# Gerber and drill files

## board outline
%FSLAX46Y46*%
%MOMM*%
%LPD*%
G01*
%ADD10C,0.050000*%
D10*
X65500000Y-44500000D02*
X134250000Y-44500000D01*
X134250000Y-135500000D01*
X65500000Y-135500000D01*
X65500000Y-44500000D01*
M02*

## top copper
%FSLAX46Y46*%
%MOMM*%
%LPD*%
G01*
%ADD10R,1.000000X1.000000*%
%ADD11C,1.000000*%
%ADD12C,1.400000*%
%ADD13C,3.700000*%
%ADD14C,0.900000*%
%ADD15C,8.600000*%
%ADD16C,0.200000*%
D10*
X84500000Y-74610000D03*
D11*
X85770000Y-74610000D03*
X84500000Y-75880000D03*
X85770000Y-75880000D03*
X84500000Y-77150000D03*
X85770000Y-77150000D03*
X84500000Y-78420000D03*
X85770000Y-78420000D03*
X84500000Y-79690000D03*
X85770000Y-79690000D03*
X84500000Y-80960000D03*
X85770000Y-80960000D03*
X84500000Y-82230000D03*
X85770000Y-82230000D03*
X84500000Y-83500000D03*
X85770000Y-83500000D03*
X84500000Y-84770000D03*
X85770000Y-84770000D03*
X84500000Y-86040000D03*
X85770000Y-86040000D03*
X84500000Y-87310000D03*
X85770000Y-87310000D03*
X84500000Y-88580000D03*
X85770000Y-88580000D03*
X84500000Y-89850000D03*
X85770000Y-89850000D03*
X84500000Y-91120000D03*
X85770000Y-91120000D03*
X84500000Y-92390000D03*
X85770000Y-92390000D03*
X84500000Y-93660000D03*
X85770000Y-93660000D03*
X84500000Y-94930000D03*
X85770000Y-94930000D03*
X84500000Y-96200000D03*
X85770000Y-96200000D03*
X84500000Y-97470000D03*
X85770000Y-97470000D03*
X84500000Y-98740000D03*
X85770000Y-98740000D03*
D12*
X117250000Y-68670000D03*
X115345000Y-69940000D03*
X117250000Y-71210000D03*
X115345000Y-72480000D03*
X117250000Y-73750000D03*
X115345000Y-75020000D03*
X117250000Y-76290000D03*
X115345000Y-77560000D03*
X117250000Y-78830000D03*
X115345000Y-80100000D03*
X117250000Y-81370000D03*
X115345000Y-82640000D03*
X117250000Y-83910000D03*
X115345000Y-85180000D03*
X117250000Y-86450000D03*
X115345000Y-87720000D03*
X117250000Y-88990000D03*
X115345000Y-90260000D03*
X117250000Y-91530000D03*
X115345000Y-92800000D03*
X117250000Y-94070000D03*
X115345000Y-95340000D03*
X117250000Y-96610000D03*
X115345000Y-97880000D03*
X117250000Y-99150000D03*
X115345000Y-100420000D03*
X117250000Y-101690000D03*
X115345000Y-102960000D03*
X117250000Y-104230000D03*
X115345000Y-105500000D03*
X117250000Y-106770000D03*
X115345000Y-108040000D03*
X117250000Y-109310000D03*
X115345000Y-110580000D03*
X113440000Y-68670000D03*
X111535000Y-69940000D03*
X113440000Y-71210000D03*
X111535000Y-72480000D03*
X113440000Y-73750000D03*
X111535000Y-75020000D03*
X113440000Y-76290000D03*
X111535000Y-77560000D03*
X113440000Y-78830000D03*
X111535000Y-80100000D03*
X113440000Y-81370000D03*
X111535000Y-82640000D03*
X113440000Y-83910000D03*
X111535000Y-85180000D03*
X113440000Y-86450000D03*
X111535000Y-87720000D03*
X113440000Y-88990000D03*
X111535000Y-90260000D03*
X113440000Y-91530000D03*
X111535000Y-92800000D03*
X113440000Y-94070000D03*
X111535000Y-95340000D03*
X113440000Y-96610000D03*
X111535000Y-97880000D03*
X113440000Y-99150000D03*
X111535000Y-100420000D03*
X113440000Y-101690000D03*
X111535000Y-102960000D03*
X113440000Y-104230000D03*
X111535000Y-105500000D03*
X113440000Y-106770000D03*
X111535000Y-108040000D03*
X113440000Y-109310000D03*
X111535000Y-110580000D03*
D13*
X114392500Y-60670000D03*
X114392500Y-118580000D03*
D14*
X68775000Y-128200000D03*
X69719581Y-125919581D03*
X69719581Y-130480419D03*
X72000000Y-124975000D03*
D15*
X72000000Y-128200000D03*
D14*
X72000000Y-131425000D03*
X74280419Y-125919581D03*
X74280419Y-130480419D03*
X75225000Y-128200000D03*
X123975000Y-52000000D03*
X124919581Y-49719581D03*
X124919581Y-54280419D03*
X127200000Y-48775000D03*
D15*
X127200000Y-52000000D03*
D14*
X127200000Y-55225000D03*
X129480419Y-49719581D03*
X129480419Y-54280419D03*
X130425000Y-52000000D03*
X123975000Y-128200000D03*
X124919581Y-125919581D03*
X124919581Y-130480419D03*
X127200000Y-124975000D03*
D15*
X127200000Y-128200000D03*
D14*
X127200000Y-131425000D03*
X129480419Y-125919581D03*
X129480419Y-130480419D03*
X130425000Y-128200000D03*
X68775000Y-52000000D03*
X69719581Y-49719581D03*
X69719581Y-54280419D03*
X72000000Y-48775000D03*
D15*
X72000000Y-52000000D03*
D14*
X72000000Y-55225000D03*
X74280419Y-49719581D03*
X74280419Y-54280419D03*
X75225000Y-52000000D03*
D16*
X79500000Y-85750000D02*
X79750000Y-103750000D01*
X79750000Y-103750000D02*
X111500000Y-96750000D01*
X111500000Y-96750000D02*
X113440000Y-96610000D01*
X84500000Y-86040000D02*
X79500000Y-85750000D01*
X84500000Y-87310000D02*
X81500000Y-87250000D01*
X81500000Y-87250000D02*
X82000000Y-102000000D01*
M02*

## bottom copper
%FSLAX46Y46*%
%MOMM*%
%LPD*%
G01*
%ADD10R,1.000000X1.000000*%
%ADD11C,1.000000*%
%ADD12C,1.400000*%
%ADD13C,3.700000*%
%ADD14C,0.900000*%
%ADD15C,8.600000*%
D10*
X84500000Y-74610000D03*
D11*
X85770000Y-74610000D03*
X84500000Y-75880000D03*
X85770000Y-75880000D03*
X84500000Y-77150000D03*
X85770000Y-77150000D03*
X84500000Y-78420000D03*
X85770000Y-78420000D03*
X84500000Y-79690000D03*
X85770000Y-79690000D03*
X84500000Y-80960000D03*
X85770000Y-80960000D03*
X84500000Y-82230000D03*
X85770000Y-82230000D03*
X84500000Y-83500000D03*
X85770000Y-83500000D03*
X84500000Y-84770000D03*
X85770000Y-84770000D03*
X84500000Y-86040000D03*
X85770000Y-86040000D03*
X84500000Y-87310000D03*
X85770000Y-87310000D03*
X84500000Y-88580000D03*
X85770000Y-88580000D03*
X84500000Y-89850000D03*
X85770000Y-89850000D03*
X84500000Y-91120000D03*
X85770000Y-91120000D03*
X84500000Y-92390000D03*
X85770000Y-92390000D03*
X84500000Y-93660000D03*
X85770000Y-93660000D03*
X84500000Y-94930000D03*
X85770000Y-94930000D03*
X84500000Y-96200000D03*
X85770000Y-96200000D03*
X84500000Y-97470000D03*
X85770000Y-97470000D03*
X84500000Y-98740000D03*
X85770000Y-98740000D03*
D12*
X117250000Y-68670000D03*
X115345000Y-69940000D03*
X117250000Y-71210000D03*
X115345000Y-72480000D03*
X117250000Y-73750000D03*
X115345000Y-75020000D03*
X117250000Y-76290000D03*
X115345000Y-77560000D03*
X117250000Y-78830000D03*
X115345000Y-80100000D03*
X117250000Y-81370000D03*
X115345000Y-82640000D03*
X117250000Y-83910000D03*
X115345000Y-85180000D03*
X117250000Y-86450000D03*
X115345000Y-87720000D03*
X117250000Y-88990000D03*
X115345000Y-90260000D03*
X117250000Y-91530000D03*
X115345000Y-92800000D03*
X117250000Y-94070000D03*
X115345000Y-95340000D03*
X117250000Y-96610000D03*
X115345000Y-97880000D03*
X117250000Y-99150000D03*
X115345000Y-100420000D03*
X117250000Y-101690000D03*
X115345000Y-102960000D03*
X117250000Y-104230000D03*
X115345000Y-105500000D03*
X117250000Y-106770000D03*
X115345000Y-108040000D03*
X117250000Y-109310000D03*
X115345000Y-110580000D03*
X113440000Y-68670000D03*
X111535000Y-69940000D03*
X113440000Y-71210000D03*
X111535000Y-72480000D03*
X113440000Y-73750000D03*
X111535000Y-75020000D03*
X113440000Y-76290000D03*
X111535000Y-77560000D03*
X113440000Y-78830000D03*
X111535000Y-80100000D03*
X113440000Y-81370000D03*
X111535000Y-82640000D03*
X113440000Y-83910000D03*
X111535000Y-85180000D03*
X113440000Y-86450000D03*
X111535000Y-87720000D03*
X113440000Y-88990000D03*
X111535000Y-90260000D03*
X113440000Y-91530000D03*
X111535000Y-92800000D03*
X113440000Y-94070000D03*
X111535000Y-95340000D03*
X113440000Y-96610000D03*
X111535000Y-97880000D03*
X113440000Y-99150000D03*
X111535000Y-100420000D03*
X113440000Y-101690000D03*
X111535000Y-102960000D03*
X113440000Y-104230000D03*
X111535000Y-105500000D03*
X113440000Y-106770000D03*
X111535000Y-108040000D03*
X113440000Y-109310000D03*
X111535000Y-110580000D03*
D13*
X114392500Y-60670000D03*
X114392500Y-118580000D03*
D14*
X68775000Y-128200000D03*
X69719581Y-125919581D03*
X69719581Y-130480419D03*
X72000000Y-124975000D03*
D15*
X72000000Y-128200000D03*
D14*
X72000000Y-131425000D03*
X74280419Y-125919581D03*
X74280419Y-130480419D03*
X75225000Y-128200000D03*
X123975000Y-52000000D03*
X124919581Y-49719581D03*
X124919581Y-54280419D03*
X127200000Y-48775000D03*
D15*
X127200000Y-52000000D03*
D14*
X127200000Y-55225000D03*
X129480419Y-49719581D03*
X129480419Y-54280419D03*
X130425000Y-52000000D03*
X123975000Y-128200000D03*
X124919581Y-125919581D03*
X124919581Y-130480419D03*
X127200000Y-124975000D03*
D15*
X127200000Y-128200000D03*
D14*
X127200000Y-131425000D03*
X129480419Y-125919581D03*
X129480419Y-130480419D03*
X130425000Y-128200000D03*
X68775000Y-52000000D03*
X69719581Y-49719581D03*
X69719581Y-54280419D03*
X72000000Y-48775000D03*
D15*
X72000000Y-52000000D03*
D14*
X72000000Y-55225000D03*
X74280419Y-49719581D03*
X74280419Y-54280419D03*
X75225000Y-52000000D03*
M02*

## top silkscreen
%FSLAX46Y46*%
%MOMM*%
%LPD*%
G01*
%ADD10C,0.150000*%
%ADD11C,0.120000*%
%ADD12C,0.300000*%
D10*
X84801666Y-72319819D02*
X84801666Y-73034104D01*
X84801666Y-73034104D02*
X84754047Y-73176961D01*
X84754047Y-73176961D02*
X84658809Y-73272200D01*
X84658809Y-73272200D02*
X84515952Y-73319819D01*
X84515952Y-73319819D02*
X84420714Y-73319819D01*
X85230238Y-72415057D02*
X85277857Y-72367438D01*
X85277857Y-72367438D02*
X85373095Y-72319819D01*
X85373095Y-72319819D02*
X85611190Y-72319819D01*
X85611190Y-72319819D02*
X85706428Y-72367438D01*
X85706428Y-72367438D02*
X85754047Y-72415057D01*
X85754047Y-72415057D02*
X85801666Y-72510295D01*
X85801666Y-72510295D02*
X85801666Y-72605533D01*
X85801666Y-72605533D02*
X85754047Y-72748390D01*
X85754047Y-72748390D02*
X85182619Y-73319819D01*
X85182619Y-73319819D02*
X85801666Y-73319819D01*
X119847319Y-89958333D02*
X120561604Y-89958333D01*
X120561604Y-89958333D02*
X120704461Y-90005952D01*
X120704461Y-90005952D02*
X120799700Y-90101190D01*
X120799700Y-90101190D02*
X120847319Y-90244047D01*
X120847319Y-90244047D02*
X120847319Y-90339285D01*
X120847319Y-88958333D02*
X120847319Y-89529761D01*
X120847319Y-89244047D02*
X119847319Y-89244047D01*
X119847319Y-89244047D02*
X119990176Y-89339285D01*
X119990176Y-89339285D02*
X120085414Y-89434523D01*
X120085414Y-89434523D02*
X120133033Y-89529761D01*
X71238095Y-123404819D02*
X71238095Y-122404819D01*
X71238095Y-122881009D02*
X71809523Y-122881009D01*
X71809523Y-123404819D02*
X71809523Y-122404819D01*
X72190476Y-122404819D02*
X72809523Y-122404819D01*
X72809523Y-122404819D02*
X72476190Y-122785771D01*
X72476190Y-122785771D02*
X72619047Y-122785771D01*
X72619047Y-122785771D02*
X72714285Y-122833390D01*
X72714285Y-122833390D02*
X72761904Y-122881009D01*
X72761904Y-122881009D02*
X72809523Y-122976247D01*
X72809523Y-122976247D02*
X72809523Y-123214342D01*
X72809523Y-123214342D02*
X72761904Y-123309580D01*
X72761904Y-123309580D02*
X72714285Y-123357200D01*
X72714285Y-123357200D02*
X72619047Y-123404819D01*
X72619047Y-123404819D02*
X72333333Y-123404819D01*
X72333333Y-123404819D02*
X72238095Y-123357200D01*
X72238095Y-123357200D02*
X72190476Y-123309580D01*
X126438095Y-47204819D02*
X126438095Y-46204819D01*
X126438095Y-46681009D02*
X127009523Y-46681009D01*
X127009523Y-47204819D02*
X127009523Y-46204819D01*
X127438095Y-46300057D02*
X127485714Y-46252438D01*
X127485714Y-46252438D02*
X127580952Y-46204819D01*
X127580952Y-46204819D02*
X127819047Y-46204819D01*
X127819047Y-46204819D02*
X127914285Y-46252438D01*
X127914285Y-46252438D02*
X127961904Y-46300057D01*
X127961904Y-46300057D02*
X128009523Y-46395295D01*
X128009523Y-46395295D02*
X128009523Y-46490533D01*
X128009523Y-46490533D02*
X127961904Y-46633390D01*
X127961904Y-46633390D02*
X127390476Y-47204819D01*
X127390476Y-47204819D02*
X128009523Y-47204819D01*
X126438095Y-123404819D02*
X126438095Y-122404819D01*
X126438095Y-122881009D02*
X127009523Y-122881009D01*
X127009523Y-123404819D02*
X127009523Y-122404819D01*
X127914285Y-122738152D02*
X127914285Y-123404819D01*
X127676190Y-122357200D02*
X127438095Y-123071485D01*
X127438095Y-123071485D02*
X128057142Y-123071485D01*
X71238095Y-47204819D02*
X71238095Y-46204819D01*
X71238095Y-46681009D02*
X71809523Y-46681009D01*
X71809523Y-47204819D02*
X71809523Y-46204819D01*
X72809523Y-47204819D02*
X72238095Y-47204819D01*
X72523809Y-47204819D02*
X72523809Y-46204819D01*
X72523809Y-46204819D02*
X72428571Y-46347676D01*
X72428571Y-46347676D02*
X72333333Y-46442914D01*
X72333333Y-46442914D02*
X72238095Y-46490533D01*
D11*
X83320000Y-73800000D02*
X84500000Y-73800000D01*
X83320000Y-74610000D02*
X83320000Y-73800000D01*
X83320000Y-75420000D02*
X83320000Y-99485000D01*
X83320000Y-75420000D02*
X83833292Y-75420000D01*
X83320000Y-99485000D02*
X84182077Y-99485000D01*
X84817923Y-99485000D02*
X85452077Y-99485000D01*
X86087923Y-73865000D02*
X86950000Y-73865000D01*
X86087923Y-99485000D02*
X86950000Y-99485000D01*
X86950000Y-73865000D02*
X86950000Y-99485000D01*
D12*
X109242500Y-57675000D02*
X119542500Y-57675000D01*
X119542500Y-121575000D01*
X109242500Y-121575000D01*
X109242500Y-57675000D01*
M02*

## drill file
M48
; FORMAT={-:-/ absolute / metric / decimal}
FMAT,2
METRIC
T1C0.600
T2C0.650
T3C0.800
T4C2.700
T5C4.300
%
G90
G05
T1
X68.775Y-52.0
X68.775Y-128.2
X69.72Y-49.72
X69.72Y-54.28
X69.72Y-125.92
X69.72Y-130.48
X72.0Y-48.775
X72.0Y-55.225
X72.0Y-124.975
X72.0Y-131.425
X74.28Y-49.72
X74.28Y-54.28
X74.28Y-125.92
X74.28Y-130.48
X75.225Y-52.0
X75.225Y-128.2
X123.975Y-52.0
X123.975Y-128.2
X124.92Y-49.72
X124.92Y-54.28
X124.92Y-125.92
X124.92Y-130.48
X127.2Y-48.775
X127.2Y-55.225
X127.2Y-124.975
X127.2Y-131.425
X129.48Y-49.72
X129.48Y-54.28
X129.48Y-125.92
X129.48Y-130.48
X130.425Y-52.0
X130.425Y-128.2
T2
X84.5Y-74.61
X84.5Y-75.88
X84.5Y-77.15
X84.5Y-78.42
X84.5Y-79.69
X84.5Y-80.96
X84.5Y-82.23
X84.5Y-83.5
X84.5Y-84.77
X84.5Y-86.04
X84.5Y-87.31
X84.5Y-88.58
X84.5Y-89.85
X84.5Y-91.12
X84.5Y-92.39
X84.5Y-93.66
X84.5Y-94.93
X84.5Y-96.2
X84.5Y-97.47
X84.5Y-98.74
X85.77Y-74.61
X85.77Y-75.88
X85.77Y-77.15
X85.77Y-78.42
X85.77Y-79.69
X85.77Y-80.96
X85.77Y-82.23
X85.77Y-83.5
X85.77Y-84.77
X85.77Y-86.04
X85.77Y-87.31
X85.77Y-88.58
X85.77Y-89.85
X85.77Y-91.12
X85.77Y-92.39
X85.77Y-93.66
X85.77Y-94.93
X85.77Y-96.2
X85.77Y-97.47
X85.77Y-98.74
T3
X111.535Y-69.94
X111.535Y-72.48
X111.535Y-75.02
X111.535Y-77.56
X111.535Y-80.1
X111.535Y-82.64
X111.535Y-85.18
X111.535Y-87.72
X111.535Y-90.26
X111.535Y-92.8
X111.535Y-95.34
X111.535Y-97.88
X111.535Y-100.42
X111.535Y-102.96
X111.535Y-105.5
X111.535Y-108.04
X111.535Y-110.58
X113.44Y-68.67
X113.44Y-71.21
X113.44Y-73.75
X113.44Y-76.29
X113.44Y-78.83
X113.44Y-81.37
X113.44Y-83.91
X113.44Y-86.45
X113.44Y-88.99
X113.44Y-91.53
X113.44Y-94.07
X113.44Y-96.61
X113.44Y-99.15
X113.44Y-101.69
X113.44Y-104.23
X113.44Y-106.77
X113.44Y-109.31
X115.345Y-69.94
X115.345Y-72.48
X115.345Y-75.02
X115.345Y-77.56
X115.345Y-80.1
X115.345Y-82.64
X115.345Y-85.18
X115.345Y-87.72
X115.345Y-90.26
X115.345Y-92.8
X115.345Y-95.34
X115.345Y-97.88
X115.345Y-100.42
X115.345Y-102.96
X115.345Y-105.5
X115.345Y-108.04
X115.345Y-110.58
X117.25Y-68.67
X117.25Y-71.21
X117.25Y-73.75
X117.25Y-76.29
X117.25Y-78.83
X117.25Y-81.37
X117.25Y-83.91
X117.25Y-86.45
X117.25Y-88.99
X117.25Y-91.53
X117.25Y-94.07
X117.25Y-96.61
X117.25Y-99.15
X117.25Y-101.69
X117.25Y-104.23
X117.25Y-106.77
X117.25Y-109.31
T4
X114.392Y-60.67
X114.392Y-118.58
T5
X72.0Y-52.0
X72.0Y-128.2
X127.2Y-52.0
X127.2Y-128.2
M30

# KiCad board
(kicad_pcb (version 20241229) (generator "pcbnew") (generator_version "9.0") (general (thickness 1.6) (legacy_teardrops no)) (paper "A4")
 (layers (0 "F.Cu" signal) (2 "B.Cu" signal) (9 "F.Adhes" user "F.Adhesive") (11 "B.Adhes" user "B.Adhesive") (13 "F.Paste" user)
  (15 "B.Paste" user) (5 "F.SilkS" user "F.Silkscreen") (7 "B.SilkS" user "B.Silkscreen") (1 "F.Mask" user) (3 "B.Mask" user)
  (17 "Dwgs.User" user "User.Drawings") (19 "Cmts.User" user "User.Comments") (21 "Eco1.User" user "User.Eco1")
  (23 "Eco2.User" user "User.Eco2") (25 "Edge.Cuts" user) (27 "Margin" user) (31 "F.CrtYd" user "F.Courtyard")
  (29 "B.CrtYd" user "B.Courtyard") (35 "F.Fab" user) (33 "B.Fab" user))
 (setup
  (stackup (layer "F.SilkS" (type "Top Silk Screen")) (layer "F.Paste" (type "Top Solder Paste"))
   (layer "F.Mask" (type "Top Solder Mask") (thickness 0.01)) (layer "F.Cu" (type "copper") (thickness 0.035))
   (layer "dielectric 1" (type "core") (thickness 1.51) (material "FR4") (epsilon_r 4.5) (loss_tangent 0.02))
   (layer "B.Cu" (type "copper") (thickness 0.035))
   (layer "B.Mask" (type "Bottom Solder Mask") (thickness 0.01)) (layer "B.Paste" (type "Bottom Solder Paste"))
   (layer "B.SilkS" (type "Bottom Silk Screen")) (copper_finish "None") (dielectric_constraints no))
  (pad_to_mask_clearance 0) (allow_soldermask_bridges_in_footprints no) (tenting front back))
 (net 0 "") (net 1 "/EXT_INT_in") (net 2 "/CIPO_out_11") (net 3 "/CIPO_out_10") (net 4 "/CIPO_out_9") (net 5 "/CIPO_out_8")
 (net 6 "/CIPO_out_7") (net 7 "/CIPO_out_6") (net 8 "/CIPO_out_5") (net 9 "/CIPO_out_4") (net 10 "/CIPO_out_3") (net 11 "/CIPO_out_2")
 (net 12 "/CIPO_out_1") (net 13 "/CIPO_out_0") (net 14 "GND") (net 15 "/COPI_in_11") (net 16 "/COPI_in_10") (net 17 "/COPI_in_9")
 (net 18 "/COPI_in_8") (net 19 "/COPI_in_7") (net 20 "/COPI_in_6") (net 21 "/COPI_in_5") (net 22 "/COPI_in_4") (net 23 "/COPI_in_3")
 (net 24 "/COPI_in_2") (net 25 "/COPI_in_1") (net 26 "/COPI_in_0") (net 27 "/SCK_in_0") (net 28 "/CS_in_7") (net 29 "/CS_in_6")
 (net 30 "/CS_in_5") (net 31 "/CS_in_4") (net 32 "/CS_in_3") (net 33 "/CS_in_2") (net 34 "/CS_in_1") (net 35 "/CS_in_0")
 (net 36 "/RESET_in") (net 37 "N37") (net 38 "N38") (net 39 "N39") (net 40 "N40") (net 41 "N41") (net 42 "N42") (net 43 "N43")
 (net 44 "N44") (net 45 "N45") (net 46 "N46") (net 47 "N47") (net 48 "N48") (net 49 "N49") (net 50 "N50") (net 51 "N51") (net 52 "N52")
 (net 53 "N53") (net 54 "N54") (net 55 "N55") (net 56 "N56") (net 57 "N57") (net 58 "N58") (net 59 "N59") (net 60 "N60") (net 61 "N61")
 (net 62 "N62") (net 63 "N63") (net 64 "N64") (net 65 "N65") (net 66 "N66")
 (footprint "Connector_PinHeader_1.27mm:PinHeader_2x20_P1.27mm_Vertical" (layer "F.Cu") (at 84.5 74.61)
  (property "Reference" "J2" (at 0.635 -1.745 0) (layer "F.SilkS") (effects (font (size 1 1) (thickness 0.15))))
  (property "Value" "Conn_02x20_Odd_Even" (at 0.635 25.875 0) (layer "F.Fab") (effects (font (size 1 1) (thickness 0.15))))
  (fp_line (start -1.18 -0.81) (end 0 -0.81) (stroke (width 0.12) (type solid)) (layer "F.SilkS"))
  (fp_line (start -1.18 0) (end -1.18 -0.81) (stroke (width 0.12) (type solid)) (layer "F.SilkS"))
  (fp_line (start -1.18 0.81) (end -1.18 24.875) (stroke (width 0.12) (type solid)) (layer "F.SilkS"))
  (fp_line (start -1.18 0.81) (end -0.666708 0.81) (stroke (width 0.12) (type solid)) (layer "F.SilkS"))
  (fp_line (start -1.18 24.875) (end -0.317923 24.875) (stroke (width 0.12) (type solid)) (layer "F.SilkS"))
  (fp_line (start 0.317923 24.875) (end 0.952077 24.875) (stroke (width 0.12) (type solid)) (layer "F.SilkS"))
  (fp_line (start 1.587923 -0.745) (end 2.45 -0.745) (stroke (width 0.12) (type solid)) (layer "F.SilkS"))
  (fp_line (start 1.587923 24.875) (end 2.45 24.875) (stroke (width 0.12) (type solid)) (layer "F.SilkS"))
  (fp_line (start 2.45 -0.745) (end 2.45 24.875) (stroke (width 0.12) (type solid)) (layer "F.SilkS"))
  (pad "1" thru_hole rect (at 0 0) (size 1 1) (drill 0.65) (layers "*.Cu" "*.Mask") (remove_unused_layers no) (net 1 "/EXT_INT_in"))
  (pad "2" thru_hole circle (at 1.27 0) (size 1 1) (drill 0.65) (layers "*.Cu" "*.Mask") (remove_unused_layers no) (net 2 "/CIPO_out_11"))
  (pad "3" thru_hole circle (at 0 1.27) (size 1 1) (drill 0.65) (layers "*.Cu" "*.Mask") (remove_unused_layers no) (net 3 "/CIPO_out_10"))
  (pad "4" thru_hole circle (at 1.27 1.27) (size 1 1) (drill 0.65) (layers "*.Cu" "*.Mask") (remove_unused_layers no) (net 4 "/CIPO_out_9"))
  (pad "5" thru_hole circle (at 0 2.54) (size 1 1) (drill 0.65) (layers "*.Cu" "*.Mask") (remove_unused_layers no) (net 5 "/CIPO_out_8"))
  (pad "6" thru_hole circle (at 1.27 2.54) (size 1 1) (drill 0.65) (layers "*.Cu" "*.Mask") (remove_unused_layers no) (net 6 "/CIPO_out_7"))
  (pad "7" thru_hole circle (at 0 3.81) (size 1 1) (drill 0.65) (layers "*.Cu" "*.Mask") (remove_unused_layers no) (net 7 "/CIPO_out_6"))
  (pad "8" thru_hole circle (at 1.27 3.81) (size 1 1) (drill 0.65) (layers "*.Cu" "*.Mask") (remove_unused_layers no) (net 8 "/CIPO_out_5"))
  (pad "9" thru_hole circle (at 0 5.08) (size 1 1) (drill 0.65) (layers "*.Cu" "*.Mask") (remove_unused_layers no) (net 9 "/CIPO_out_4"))
  (pad "10" thru_hole circle (at 1.27 5.08) (size 1 1) (drill 0.65) (layers "*.Cu" "*.Mask") (remove_unused_layers no)
   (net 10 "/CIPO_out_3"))
  (pad "11" thru_hole circle (at 0 6.35) (size 1 1) (drill 0.65) (layers "*.Cu" "*.Mask") (remove_unused_layers no) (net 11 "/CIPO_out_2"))
  (pad "12" thru_hole circle (at 1.27 6.35) (size 1 1) (drill 0.65) (layers "*.Cu" "*.Mask") (remove_unused_layers no)
   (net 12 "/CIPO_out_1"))
  (pad "13" thru_hole circle (at 0 7.62) (size 1 1) (drill 0.65) (layers "*.Cu" "*.Mask") (remove_unused_layers no) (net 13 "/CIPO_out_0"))
  (pad "14" thru_hole circle (at 1.27 7.62) (size 1 1) (drill 0.65) (layers "*.Cu" "*.Mask") (remove_unused_layers no) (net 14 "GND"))
  (pad "15" thru_hole circle (at 0 8.89) (size 1 1) (drill 0.65) (layers "*.Cu" "*.Mask") (remove_unused_layers no) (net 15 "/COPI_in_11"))
  (pad "16" thru_hole circle (at 1.27 8.89) (size 1 1) (drill 0.65) (layers "*.Cu" "*.Mask") (remove_unused_layers no)
   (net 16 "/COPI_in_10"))
  (pad "17" thru_hole circle (at 0 10.16) (size 1 1) (drill 0.65) (layers "*.Cu" "*.Mask") (remove_unused_layers no) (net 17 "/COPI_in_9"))
  (pad "18" thru_hole circle (at 1.27 10.16) (size 1 1) (drill 0.65) (layers "*.Cu" "*.Mask") (remove_unused_layers no)
   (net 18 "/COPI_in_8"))
  (pad "19" thru_hole circle (at 0 11.43) (size 1 1) (drill 0.65) (layers "*.Cu" "*.Mask") (remove_unused_layers no) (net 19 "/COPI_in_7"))
  (pad "20" thru_hole circle (at 1.27 11.43) (size 1 1) (drill 0.65) (layers "*.Cu" "*.Mask") (remove_unused_layers no)
   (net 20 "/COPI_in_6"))
  (pad "21" thru_hole circle (at 0 12.7) (size 1 1) (drill 0.65) (layers "*.Cu" "*.Mask") (remove_unused_layers no) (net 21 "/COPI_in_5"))
  (pad "22" thru_hole circle (at 1.27 12.7) (size 1 1) (drill 0.65) (layers "*.Cu" "*.Mask") (remove_unused_layers no) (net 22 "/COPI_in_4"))
  (pad "23" thru_hole circle (at 0 13.97) (size 1 1) (drill 0.65) (layers "*.Cu" "*.Mask") (remove_unused_layers no) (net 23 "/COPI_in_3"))
  (pad "24" thru_hole circle (at 1.27 13.97) (size 1 1) (drill 0.65) (layers "*.Cu" "*.Mask") (remove_unused_layers no)
   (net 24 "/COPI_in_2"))
  (pad "25" thru_hole circle (at 0 15.24) (size 1 1) (drill 0.65) (layers "*.Cu" "*.Mask") (remove_unused_layers no) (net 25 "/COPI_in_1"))
  (pad "26" thru_hole circle (at 1.27 15.24) (size 1 1) (drill 0.65) (layers "*.Cu" "*.Mask") (remove_unused_layers no)
   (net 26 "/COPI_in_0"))
  (pad "27" thru_hole circle (at 0 16.51) (size 1 1) (drill 0.65) (layers "*.Cu" "*.Mask") (remove_unused_layers no) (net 14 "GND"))
  (pad "28" thru_hole circle (at 1.27 16.51) (size 1 1) (drill 0.65) (layers "*.Cu" "*.Mask") (remove_unused_layers no) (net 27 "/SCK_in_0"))
  (pad "29" thru_hole circle (at 0 17.78) (size 1 1) (drill 0.65) (layers "*.Cu" "*.Mask") (remove_unused_layers no) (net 14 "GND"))
  (pad "30" thru_hole circle (at 1.27 17.78) (size 1 1) (drill 0.65) (layers "*.Cu" "*.Mask") (remove_unused_layers no) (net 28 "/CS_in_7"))
  (pad "31" thru_hole circle (at 0 19.05) (size 1 1) (drill 0.65) (layers "*.Cu" "*.Mask") (remove_unused_layers no) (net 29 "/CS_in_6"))
  (pad "32" thru_hole circle (at 1.27 19.05) (size 1 1) (drill 0.65) (layers "*.Cu" "*.Mask") (remove_unused_layers no) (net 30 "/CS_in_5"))
  (pad "33" thru_hole circle (at 0 20.32) (size 1 1) (drill 0.65) (layers "*.Cu" "*.Mask") (remove_unused_layers no) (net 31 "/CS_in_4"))
  (pad "34" thru_hole circle (at 1.27 20.32) (size 1 1) (drill 0.65) (layers "*.Cu" "*.Mask") (remove_unused_layers no) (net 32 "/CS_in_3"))
  (pad "35" thru_hole circle (at 0 21.59) (size 1 1) (drill 0.65) (layers "*.Cu" "*.Mask") (remove_unused_layers no) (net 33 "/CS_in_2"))
  (pad "36" thru_hole circle (at 1.27 21.59) (size 1 1) (drill 0.65) (layers "*.Cu" "*.Mask") (remove_unused_layers no) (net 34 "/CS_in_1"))
  (pad "37" thru_hole circle (at 0 22.86) (size 1 1) (drill 0.65) (layers "*.Cu" "*.Mask") (remove_unused_layers no) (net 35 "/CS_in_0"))
  (pad "38" thru_hole circle (at 1.27 22.86) (size 1 1) (drill 0.65) (layers "*.Cu" "*.Mask") (remove_unused_layers no) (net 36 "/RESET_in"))
  (pad "39" thru_hole circle (at 0 24.13) (size 1 1) (drill 0.65) (layers "*.Cu" "*.Mask") (remove_unused_layers no) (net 14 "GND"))
  (pad "40" thru_hole circle (at 1.27 24.13) (size 1 1) (drill 0.65) (layers "*.Cu" "*.Mask") (remove_unused_layers no) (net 14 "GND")))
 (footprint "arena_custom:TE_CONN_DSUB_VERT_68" (layer "F.Cu") (at 114.3925 89.625 -90)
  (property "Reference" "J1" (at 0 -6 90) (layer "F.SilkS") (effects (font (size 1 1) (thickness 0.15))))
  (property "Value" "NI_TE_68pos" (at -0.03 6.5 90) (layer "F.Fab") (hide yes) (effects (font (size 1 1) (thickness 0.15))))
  (fp_rect (start -31.95 -5.15) (end 31.95 5.15) (stroke (width 0.3) (type default)) (fill no) (layer "F.SilkS"))
  (pad "1" thru_hole circle (at -20.955 -2.8575 270) (size 1.4 1.4) (drill 0.8) (layers "*.Cu" "*.Mask") (remove_unused_layers no)
   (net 14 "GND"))
  (pad "2" thru_hole circle (at -19.685 -0.9525 270) (size 1.4 1.4) (drill 0.8) (layers "*.Cu" "*.Mask") (remove_unused_layers no)
   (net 14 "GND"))
  (pad "3" thru_hole circle (at -18.415 -2.8575 270) (size 1.4 1.4) (drill 0.8) (layers "*.Cu" "*.Mask") (remove_unused_layers no)
   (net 14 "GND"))
  (pad "4" thru_hole circle (at -17.145 -0.9525 270) (size 1.4 1.4) (drill 0.8) (layers "*.Cu" "*.Mask") (remove_unused_layers no)
   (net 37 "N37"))
  (pad "5" thru_hole circle (at -15.875 -2.8575 270) (size 1.4 1.4) (drill 0.8) (layers "*.Cu" "*.Mask") (remove_unused_layers no)
   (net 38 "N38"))
  (pad "6" thru_hole circle (at -14.605 -0.9525 270) (size 1.4 1.4) (drill 0.8) (layers "*.Cu" "*.Mask") (remove_unused_layers no)
   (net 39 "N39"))
  (pad "7" thru_hole circle (at -13.335 -2.8575 270) (size 1.4 1.4) (drill 0.8) (layers "*.Cu" "*.Mask") (remove_unused_layers no)
   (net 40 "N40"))
  (pad "8" thru_hole circle (at -12.065 -0.9525 270) (size 1.4 1.4) (drill 0.8) (layers "*.Cu" "*.Mask") (remove_unused_layers no)
   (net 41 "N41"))
  (pad "9" thru_hole circle (at -10.795 -2.8575 270) (size 1.4 1.4) (drill 0.8) (layers "*.Cu" "*.Mask") (remove_unused_layers no)
   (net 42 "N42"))
  (pad "10" thru_hole circle (at -9.525 -0.9525 270) (size 1.4 1.4) (drill 0.8) (layers "*.Cu" "*.Mask") (remove_unused_layers no)
   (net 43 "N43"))
  (pad "11" thru_hole circle (at -8.255 -2.8575 270) (size 1.4 1.4) (drill 0.8) (layers "*.Cu" "*.Mask") (remove_unused_layers no)
   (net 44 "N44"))
  (pad "12" thru_hole circle (at -6.985 -0.9525 270) (size 1.4 1.4) (drill 0.8) (layers "*.Cu" "*.Mask") (remove_unused_layers no)
   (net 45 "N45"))
  (pad "13" thru_hole circle (at -5.715 -2.8575 270) (size 1.4 1.4) (drill 0.8) (layers "*.Cu" "*.Mask") (remove_unused_layers no)
   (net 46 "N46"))
  (pad "14" thru_hole circle (at -4.445 -0.9525 270) (size 1.4 1.4) (drill 0.8) (layers "*.Cu" "*.Mask") (remove_unused_layers no)
   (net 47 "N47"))
  (pad "15" thru_hole circle (at -3.175 -2.8575 270) (size 1.4 1.4) (drill 0.8) (layers "*.Cu" "*.Mask") (remove_unused_layers no)
   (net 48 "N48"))
  (pad "16" thru_hole circle (at -1.905 -0.9525 270) (size 1.4 1.4) (drill 0.8) (layers "*.Cu" "*.Mask") (remove_unused_layers no)
   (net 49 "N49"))
  (pad "17" thru_hole circle (at -0.635 -2.8575 270) (size 1.4 1.4) (drill 0.8) (layers "*.Cu" "*.Mask") (remove_unused_layers no)
   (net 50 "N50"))
  (pad "18" thru_hole circle (at 0.635 -0.9525 270) (size 1.4 1.4) (drill 0.8) (layers "*.Cu" "*.Mask") (remove_unused_layers no)
   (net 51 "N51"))
  (pad "19" thru_hole circle (at 1.905 -2.8575 270) (size 1.4 1.4) (drill 0.8) (layers "*.Cu" "*.Mask") (remove_unused_layers no)
   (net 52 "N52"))
  (pad "20" thru_hole circle (at 3.175 -0.9525 270) (size 1.4 1.4) (drill 0.8) (layers "*.Cu" "*.Mask") (remove_unused_layers no)
   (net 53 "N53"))
  (pad "21" thru_hole circle (at 4.445 -2.8575 270) (size 1.4 1.4) (drill 0.8) (layers "*.Cu" "*.Mask") (remove_unused_layers no)
   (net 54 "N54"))
  (pad "22" thru_hole circle (at 5.715 -0.9525 270) (size 1.4 1.4) (drill 0.8) (layers "*.Cu" "*.Mask") (remove_unused_layers no)
   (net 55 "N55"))
  (pad "23" thru_hole circle (at 6.985 -2.8575 270) (size 1.4 1.4) (drill 0.8) (layers "*.Cu" "*.Mask") (remove_unused_layers no)
   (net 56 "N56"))
  (pad "24" thru_hole circle (at 8.255 -0.9525 270) (size 1.4 1.4) (drill 0.8) (layers "*.Cu" "*.Mask") (remove_unused_layers no)
   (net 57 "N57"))
  (pad "25" thru_hole circle (at 9.525 -2.8575 270) (size 1.4 1.4) (drill 0.8) (layers "*.Cu" "*.Mask") (remove_unused_layers no)
   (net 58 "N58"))
  (pad "26" thru_hole circle (at 10.795 -0.9525 270) (size 1.4 1.4) (drill 0.8) (layers "*.Cu" "*.Mask") (remove_unused_layers no)
   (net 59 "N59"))
  (pad "27" thru_hole circle (at 12.065 -2.8575 270) (size 1.4 1.4) (drill 0.8) (layers "*.Cu" "*.Mask") (remove_unused_layers no)
   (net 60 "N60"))
  (pad "28" thru_hole circle (at 13.335 -0.9525 270) (size 1.4 1.4) (drill 0.8) (layers "*.Cu" "*.Mask") (remove_unused_layers no)
   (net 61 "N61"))
  (pad "29" thru_hole circle (at 14.605 -2.8575 270) (size 1.4 1.4) (drill 0.8) (layers "*.Cu" "*.Mask") (remove_unused_layers no)
   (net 22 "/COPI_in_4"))
  (pad "30" thru_hole circle (at 15.875 -0.9525 270) (size 1.4 1.4) (drill 0.8) (layers "*.Cu" "*.Mask") (remove_unused_layers no)
   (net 23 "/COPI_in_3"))
  (pad "31" thru_hole circle (at 17.145 -2.8575 270) (size 1.4 1.4) (drill 0.8) (layers "*.Cu" "*.Mask") (remove_unused_layers no)
   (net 24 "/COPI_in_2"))
  (pad "32" thru_hole circle (at 18.415 -0.9525 270) (size 1.4 1.4) (drill 0.8) (layers "*.Cu" "*.Mask") (remove_unused_layers no)
   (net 25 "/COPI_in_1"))
  (pad "33" thru_hole circle (at 19.685 -2.8575 270) (size 1.4 1.4) (drill 0.8) (layers "*.Cu" "*.Mask") (remove_unused_layers no)
   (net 26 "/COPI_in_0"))
  (pad "34" thru_hole circle (at 20.955 -0.9525 270) (size 1.4 1.4) (drill 0.8) (layers "*.Cu" "*.Mask") (remove_unused_layers no)
   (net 36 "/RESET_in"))
  (pad "35" thru_hole circle (at -20.955 0.9525 270) (size 1.4 1.4) (drill 0.8) (layers "*.Cu" "*.Mask") (remove_unused_layers no)
   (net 35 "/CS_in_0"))
  (pad "36" thru_hole circle (at -19.685 2.8575 270) (size 1.4 1.4) (drill 0.8) (layers "*.Cu" "*.Mask") (remove_unused_layers no)
   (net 34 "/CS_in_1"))
  (pad "37" thru_hole circle (at -18.415 0.9525 270) (size 1.4 1.4) (drill 0.8) (layers "*.Cu" "*.Mask") (remove_unused_layers no)
   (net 33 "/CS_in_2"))
  (pad "38" thru_hole circle (at -17.145 2.8575 270) (size 1.4 1.4) (drill 0.8) (layers "*.Cu" "*.Mask") (remove_unused_layers no)
   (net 32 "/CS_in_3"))
  (pad "39" thru_hole circle (at -15.875 0.9525 270) (size 1.4 1.4) (drill 0.8) (layers "*.Cu" "*.Mask") (remove_unused_layers no)
   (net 31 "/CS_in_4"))
  (pad "40" thru_hole circle (at -14.605 2.8575 270) (size 1.4 1.4) (drill 0.8) (layers "*.Cu" "*.Mask") (remove_unused_layers no)
   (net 30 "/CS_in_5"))
  (pad "41" thru_hole circle (at -13.335 0.9525 270) (size 1.4 1.4) (drill 0.8) (layers "*.Cu" "*.Mask") (remove_unused_layers no)
   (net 29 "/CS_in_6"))
  (pad "42" thru_hole circle (at -12.065 2.8575 270) (size 1.4 1.4) (drill 0.8) (layers "*.Cu" "*.Mask") (remove_unused_layers no)
   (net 28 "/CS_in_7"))
  (pad "43" thru_hole circle (at -10.795 0.9525 270) (size 1.4 1.4) (drill 0.8) (layers "*.Cu" "*.Mask") (remove_unused_layers no)
   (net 27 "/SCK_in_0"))
  (pad "44" thru_hole circle (at -9.525 2.8575 270) (size 1.4 1.4) (drill 0.8) (layers "*.Cu" "*.Mask") (remove_unused_layers no)
   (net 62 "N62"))
  (pad "45" thru_hole circle (at -8.255 0.9525 270) (size 1.4 1.4) (drill 0.8) (layers "*.Cu" "*.Mask") (remove_unused_layers no)
   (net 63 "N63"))
  (pad "46" thru_hole circle (at -6.985 2.8575 270) (size 1.4 1.4) (drill 0.8) (layers "*.Cu" "*.Mask") (remove_unused_layers no)
   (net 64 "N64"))
  (pad "47" thru_hole circle (at -5.715 0.9525 270) (size 1.4 1.4) (drill 0.8) (layers "*.Cu" "*.Mask") (remove_unused_layers no)
   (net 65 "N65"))
  (pad "48" thru_hole circle (at -4.445 2.8575 270) (size 1.4 1.4) (drill 0.8) (layers "*.Cu" "*.Mask") (remove_unused_layers no)
   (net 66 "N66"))
  (pad "49" thru_hole circle (at -3.175 0.9525 270) (size 1.4 1.4) (drill 0.8) (layers "*.Cu" "*.Mask") (remove_unused_layers no)
   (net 15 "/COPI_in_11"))
  (pad "50" thru_hole circle (at -1.905 2.8575 270) (size 1.4 1.4) (drill 0.8) (layers "*.Cu" "*.Mask") (remove_unused_layers no)
   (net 2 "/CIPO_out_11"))
  (pad "51" thru_hole circle (at -0.635 0.9525 270) (size 1.4 1.4) (drill 0.8) (layers "*.Cu" "*.Mask") (remove_unused_layers no)
   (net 16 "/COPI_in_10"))
  (pad "52" thru_hole circle (at 0.635 2.8575 270) (size 1.4 1.4) (drill 0.8) (layers "*.Cu" "*.Mask") (remove_unused_layers no)
   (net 3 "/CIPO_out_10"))
  (pad "53" thru_hole circle (at 1.905 0.9525 270) (size 1.4 1.4) (drill 0.8) (layers "*.Cu" "*.Mask") (remove_unused_layers no)
   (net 17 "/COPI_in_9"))
  (pad "54" thru_hole circle (at 3.175 2.8575 270) (size 1.4 1.4) (drill 0.8) (layers "*.Cu" "*.Mask") (remove_unused_layers no)
   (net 4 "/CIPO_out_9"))
  (pad "55" thru_hole circle (at 4.445 0.9525 270) (size 1.4 1.4) (drill 0.8) (layers "*.Cu" "*.Mask") (remove_unused_layers no)
   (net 18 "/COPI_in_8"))
  (pad "56" thru_hole circle (at 5.715 2.8575 270) (size 1.4 1.4) (drill 0.8) (layers "*.Cu" "*.Mask") (remove_unused_layers no)
   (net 5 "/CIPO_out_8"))
  (pad "57" thru_hole circle (at 6.985 0.9525 270) (size 1.4 1.4) (drill 0.8) (layers "*.Cu" "*.Mask") (remove_unused_layers no)
   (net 19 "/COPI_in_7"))
  (pad "58" thru_hole circle (at 8.255 2.8575 270) (size 1.4 1.4) (drill 0.8) (layers "*.Cu" "*.Mask") (remove_unused_layers no)
   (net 6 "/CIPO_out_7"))
  (pad "59" thru_hole circle (at 9.525 0.9525 270) (size 1.4 1.4) (drill 0.8) (layers "*.Cu" "*.Mask") (remove_unused_layers no)
   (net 20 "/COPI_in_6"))
  (pad "60" thru_hole circle (at 10.795 2.8575 270) (size 1.4 1.4) (drill 0.8) (layers "*.Cu" "*.Mask") (remove_unused_layers no)
   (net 7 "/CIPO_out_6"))
  (pad "61" thru_hole circle (at 12.065 0.9525 270) (size 1.4 1.4) (drill 0.8) (layers "*.Cu" "*.Mask") (remove_unused_layers no)
   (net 21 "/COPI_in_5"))
  (pad "62" thru_hole circle (at 13.335 2.8575 270) (size 1.4 1.4) (drill 0.8) (layers "*.Cu" "*.Mask") (remove_unused_layers no)
   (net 8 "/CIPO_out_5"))
  (pad "63" thru_hole circle (at 14.605 0.9525 270) (size 1.4 1.4) (drill 0.8) (layers "*.Cu" "*.Mask") (remove_unused_layers no)
   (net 9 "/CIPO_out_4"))
  (pad "64" thru_hole circle (at 15.875 2.8575 270) (size 1.4 1.4) (drill 0.8) (layers "*.Cu" "*.Mask") (remove_unused_layers no)
   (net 10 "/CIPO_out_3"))
  (pad "65" thru_hole circle (at 17.145 0.9525 270) (size 1.4 1.4) (drill 0.8) (layers "*.Cu" "*.Mask") (remove_unused_layers no)
   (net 11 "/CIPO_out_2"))
  (pad "66" thru_hole circle (at 18.415 2.8575 270) (size 1.4 1.4) (drill 0.8) (layers "*.Cu" "*.Mask") (remove_unused_layers no)
   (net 12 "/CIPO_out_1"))
  (pad "67" thru_hole circle (at 19.685 0.9525 270) (size 1.4 1.4) (drill 0.8) (layers "*.Cu" "*.Mask") (remove_unused_layers no)
   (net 13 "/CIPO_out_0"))
  (pad "68" thru_hole circle (at 20.955 2.8575 270) (size 1.4 1.4) (drill 0.8) (layers "*.Cu" "*.Mask") (remove_unused_layers no)
   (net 1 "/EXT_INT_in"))
  (pad "69" thru_hole circle (at -28.955 0 270) (size 3.7 3.7) (drill 2.7) (layers "*.Cu" "*.Mask") (remove_unused_layers no) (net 14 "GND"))
  (pad "70" thru_hole circle (at 28.955 0 270) (size 3.7 3.7) (drill 2.7) (layers "*.Cu" "*.Mask") (remove_unused_layers no) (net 14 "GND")))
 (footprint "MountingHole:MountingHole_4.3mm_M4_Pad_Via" (layer "F.Cu") (at 72 128.2)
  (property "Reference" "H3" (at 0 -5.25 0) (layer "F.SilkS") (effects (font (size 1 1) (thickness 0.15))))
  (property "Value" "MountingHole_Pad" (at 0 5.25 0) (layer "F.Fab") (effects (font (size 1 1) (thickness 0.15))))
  (pad "1" thru_hole circle (at -3.225 0) (size 0.9 0.9) (drill 0.6) (layers "*.Cu" "*.Mask") (remove_unused_layers no) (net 14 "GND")
   (zone_connect 2))
  (pad "1" thru_hole circle (at -2.280419 -2.280419) (size 0.9 0.9) (drill 0.6) (layers "*.Cu" "*.Mask") (remove_unused_layers no)
   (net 14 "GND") (zone_connect 2))
  (pad "1" thru_hole circle (at -2.280419 2.280419) (size 0.9 0.9) (drill 0.6) (layers "*.Cu" "*.Mask") (remove_unused_layers no)
   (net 14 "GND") (zone_connect 2))
  (pad "1" thru_hole circle (at 0 -3.225) (size 0.9 0.9) (drill 0.6) (layers "*.Cu" "*.Mask") (remove_unused_layers no) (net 14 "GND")
   (zone_connect 2))
  (pad "1" thru_hole circle (at 0 0) (size 8.6 8.6) (drill 4.3) (layers "*.Cu" "*.Mask") (remove_unused_layers no) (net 14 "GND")
   (zone_connect 2))
  (pad "1" thru_hole circle (at 0 3.225) (size 0.9 0.9) (drill 0.6) (layers "*.Cu" "*.Mask") (remove_unused_layers no) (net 14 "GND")
   (zone_connect 2))
  (pad "1" thru_hole circle (at 2.280419 -2.280419) (size 0.9 0.9) (drill 0.6) (layers "*.Cu" "*.Mask") (remove_unused_layers no)
   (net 14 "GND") (zone_connect 2))
  (pad "1" thru_hole circle (at 2.280419 2.280419) (size 0.9 0.9) (drill 0.6) (layers "*.Cu" "*.Mask") (remove_unused_layers no)
   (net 14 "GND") (zone_connect 2))
  (pad "1" thru_hole circle (at 3.225 0) (size 0.9 0.9) (drill 0.6) (layers "*.Cu" "*.Mask") (remove_unused_layers no) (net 14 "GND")
   (zone_connect 2)))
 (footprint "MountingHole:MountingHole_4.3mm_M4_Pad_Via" (layer "F.Cu") (at 127.2 52)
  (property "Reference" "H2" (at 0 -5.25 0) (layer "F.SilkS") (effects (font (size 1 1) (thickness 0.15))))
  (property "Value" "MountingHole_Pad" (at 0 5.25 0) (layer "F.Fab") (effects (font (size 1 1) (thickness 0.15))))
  (pad "1" thru_hole circle (at -3.225 0) (size 0.9 0.9) (drill 0.6) (layers "*.Cu" "*.Mask") (remove_unused_layers no) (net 14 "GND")
   (zone_connect 2))
  (pad "1" thru_hole circle (at -2.280419 -2.280419) (size 0.9 0.9) (drill 0.6) (layers "*.Cu" "*.Mask") (remove_unused_layers no)
   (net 14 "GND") (zone_connect 2))
  (pad "1" thru_hole circle (at -2.280419 2.280419) (size 0.9 0.9) (drill 0.6) (layers "*.Cu" "*.Mask") (remove_unused_layers no)
   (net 14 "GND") (zone_connect 2))
  (pad "1" thru_hole circle (at 0 -3.225) (size 0.9 0.9) (drill 0.6) (layers "*.Cu" "*.Mask") (remove_unused_layers no) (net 14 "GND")
   (zone_connect 2))
  (pad "1" thru_hole circle (at 0 0) (size 8.6 8.6) (drill 4.3) (layers "*.Cu" "*.Mask") (remove_unused_layers no) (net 14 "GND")
   (zone_connect 2))
  (pad "1" thru_hole circle (at 0 3.225) (size 0.9 0.9) (drill 0.6) (layers "*.Cu" "*.Mask") (remove_unused_layers no) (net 14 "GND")
   (zone_connect 2))
  (pad "1" thru_hole circle (at 2.280419 -2.280419) (size 0.9 0.9) (drill 0.6) (layers "*.Cu" "*.Mask") (remove_unused_layers no)
   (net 14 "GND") (zone_connect 2))
  (pad "1" thru_hole circle (at 2.280419 2.280419) (size 0.9 0.9) (drill 0.6) (layers "*.Cu" "*.Mask") (remove_unused_layers no)
   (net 14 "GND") (zone_connect 2))
  (pad "1" thru_hole circle (at 3.225 0) (size 0.9 0.9) (drill 0.6) (layers "*.Cu" "*.Mask") (remove_unused_layers no) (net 14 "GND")
   (zone_connect 2)))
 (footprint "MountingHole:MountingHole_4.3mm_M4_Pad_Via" (layer "F.Cu") (at 127.2 128.2)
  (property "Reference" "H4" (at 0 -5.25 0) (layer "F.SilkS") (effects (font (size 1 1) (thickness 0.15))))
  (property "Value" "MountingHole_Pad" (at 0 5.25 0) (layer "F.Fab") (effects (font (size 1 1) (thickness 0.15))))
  (pad "1" thru_hole circle (at -3.225 0) (size 0.9 0.9) (drill 0.6) (layers "*.Cu" "*.Mask") (remove_unused_layers no) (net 14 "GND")
   (zone_connect 2))
  (pad "1" thru_hole circle (at -2.280419 -2.280419) (size 0.9 0.9) (drill 0.6) (layers "*.Cu" "*.Mask") (remove_unused_layers no)
   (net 14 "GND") (zone_connect 2))
  (pad "1" thru_hole circle (at -2.280419 2.280419) (size 0.9 0.9) (drill 0.6) (layers "*.Cu" "*.Mask") (remove_unused_layers no)
   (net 14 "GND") (zone_connect 2))
  (pad "1" thru_hole circle (at 0 -3.225) (size 0.9 0.9) (drill 0.6) (layers "*.Cu" "*.Mask") (remove_unused_layers no) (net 14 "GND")
   (zone_connect 2))
  (pad "1" thru_hole circle (at 0 0) (size 8.6 8.6) (drill 4.3) (layers "*.Cu" "*.Mask") (remove_unused_layers no) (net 14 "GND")
   (zone_connect 2))
  (pad "1" thru_hole circle (at 0 3.225) (size 0.9 0.9) (drill 0.6) (layers "*.Cu" "*.Mask") (remove_unused_layers no) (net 14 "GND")
   (zone_connect 2))
  (pad "1" thru_hole circle (at 2.280419 -2.280419) (size 0.9 0.9) (drill 0.6) (layers "*.Cu" "*.Mask") (remove_unused_layers no)
   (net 14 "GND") (zone_connect 2))
  (pad "1" thru_hole circle (at 2.280419 2.280419) (size 0.9 0.9) (drill 0.6) (layers "*.Cu" "*.Mask") (remove_unused_layers no)
   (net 14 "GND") (zone_connect 2))
  (pad "1" thru_hole circle (at 3.225 0) (size 0.9 0.9) (drill 0.6) (layers "*.Cu" "*.Mask") (remove_unused_layers no) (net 14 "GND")
   (zone_connect 2)))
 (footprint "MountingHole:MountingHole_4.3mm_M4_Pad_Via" (layer "F.Cu") (at 72 52)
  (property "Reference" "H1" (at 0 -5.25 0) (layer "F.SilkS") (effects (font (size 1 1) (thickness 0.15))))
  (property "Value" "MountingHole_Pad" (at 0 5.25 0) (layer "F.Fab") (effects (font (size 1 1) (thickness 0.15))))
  (pad "1" thru_hole circle (at -3.225 0) (size 0.9 0.9) (drill 0.6) (layers "*.Cu" "*.Mask") (remove_unused_layers no) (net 14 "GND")
   (zone_connect 2))
  (pad "1" thru_hole circle (at -2.280419 -2.280419) (size 0.9 0.9) (drill 0.6) (layers "*.Cu" "*.Mask") (remove_unused_layers no)
   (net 14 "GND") (zone_connect 2))
  (pad "1" thru_hole circle (at -2.280419 2.280419) (size 0.9 0.9) (drill 0.6) (layers "*.Cu" "*.Mask") (remove_unused_layers no)
   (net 14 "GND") (zone_connect 2))
  (pad "1" thru_hole circle (at 0 -3.225) (size 0.9 0.9) (drill 0.6) (layers "*.Cu" "*.Mask") (remove_unused_layers no) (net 14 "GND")
   (zone_connect 2))
  (pad "1" thru_hole circle (at 0 0) (size 8.6 8.6) (drill 4.3) (layers "*.Cu" "*.Mask") (remove_unused_layers no) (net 14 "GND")
   (zone_connect 2))
  (pad "1" thru_hole circle (at 0 3.225) (size 0.9 0.9) (drill 0.6) (layers "*.Cu" "*.Mask") (remove_unused_layers no) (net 14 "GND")
   (zone_connect 2))
  (pad "1" thru_hole circle (at 2.280419 -2.280419) (size 0.9 0.9) (drill 0.6) (layers "*.Cu" "*.Mask") (remove_unused_layers no)
   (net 14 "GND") (zone_connect 2))
  (pad "1" thru_hole circle (at 2.280419 2.280419) (size 0.9 0.9) (drill 0.6) (layers "*.Cu" "*.Mask") (remove_unused_layers no)
   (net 14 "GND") (zone_connect 2))
  (pad "1" thru_hole circle (at 3.225 0) (size 0.9 0.9) (drill 0.6) (layers "*.Cu" "*.Mask") (remove_unused_layers no) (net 14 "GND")
   (zone_connect 2)))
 (gr_rect (start 65.5 44.5) (end 134.25 135.5) (stroke (width 0.05) (type default)) (fill no) (layer "Edge.Cuts"))
 (segment (start 79.5 85.75) (end 79.75 103.75) (width 0.2) (layer "F.Cu") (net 19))
 (segment (start 79.75 103.75) (end 111.5 96.75) (width 0.2) (layer "F.Cu") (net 19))
 (segment (start 111.5 96.75) (end 113.44 96.61) (width 0.2) (layer "F.Cu") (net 19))
 (segment (start 84.5 86.04) (end 79.5 85.75) (width 0.2) (layer "F.Cu") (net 19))
 (segment (start 84.5 87.31) (end 81.5 87.25) (width 0.2) (layer "F.Cu") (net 21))
 (segment (start 81.5 87.25) (end 82 102) (width 0.2) (layer "F.Cu") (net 21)))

